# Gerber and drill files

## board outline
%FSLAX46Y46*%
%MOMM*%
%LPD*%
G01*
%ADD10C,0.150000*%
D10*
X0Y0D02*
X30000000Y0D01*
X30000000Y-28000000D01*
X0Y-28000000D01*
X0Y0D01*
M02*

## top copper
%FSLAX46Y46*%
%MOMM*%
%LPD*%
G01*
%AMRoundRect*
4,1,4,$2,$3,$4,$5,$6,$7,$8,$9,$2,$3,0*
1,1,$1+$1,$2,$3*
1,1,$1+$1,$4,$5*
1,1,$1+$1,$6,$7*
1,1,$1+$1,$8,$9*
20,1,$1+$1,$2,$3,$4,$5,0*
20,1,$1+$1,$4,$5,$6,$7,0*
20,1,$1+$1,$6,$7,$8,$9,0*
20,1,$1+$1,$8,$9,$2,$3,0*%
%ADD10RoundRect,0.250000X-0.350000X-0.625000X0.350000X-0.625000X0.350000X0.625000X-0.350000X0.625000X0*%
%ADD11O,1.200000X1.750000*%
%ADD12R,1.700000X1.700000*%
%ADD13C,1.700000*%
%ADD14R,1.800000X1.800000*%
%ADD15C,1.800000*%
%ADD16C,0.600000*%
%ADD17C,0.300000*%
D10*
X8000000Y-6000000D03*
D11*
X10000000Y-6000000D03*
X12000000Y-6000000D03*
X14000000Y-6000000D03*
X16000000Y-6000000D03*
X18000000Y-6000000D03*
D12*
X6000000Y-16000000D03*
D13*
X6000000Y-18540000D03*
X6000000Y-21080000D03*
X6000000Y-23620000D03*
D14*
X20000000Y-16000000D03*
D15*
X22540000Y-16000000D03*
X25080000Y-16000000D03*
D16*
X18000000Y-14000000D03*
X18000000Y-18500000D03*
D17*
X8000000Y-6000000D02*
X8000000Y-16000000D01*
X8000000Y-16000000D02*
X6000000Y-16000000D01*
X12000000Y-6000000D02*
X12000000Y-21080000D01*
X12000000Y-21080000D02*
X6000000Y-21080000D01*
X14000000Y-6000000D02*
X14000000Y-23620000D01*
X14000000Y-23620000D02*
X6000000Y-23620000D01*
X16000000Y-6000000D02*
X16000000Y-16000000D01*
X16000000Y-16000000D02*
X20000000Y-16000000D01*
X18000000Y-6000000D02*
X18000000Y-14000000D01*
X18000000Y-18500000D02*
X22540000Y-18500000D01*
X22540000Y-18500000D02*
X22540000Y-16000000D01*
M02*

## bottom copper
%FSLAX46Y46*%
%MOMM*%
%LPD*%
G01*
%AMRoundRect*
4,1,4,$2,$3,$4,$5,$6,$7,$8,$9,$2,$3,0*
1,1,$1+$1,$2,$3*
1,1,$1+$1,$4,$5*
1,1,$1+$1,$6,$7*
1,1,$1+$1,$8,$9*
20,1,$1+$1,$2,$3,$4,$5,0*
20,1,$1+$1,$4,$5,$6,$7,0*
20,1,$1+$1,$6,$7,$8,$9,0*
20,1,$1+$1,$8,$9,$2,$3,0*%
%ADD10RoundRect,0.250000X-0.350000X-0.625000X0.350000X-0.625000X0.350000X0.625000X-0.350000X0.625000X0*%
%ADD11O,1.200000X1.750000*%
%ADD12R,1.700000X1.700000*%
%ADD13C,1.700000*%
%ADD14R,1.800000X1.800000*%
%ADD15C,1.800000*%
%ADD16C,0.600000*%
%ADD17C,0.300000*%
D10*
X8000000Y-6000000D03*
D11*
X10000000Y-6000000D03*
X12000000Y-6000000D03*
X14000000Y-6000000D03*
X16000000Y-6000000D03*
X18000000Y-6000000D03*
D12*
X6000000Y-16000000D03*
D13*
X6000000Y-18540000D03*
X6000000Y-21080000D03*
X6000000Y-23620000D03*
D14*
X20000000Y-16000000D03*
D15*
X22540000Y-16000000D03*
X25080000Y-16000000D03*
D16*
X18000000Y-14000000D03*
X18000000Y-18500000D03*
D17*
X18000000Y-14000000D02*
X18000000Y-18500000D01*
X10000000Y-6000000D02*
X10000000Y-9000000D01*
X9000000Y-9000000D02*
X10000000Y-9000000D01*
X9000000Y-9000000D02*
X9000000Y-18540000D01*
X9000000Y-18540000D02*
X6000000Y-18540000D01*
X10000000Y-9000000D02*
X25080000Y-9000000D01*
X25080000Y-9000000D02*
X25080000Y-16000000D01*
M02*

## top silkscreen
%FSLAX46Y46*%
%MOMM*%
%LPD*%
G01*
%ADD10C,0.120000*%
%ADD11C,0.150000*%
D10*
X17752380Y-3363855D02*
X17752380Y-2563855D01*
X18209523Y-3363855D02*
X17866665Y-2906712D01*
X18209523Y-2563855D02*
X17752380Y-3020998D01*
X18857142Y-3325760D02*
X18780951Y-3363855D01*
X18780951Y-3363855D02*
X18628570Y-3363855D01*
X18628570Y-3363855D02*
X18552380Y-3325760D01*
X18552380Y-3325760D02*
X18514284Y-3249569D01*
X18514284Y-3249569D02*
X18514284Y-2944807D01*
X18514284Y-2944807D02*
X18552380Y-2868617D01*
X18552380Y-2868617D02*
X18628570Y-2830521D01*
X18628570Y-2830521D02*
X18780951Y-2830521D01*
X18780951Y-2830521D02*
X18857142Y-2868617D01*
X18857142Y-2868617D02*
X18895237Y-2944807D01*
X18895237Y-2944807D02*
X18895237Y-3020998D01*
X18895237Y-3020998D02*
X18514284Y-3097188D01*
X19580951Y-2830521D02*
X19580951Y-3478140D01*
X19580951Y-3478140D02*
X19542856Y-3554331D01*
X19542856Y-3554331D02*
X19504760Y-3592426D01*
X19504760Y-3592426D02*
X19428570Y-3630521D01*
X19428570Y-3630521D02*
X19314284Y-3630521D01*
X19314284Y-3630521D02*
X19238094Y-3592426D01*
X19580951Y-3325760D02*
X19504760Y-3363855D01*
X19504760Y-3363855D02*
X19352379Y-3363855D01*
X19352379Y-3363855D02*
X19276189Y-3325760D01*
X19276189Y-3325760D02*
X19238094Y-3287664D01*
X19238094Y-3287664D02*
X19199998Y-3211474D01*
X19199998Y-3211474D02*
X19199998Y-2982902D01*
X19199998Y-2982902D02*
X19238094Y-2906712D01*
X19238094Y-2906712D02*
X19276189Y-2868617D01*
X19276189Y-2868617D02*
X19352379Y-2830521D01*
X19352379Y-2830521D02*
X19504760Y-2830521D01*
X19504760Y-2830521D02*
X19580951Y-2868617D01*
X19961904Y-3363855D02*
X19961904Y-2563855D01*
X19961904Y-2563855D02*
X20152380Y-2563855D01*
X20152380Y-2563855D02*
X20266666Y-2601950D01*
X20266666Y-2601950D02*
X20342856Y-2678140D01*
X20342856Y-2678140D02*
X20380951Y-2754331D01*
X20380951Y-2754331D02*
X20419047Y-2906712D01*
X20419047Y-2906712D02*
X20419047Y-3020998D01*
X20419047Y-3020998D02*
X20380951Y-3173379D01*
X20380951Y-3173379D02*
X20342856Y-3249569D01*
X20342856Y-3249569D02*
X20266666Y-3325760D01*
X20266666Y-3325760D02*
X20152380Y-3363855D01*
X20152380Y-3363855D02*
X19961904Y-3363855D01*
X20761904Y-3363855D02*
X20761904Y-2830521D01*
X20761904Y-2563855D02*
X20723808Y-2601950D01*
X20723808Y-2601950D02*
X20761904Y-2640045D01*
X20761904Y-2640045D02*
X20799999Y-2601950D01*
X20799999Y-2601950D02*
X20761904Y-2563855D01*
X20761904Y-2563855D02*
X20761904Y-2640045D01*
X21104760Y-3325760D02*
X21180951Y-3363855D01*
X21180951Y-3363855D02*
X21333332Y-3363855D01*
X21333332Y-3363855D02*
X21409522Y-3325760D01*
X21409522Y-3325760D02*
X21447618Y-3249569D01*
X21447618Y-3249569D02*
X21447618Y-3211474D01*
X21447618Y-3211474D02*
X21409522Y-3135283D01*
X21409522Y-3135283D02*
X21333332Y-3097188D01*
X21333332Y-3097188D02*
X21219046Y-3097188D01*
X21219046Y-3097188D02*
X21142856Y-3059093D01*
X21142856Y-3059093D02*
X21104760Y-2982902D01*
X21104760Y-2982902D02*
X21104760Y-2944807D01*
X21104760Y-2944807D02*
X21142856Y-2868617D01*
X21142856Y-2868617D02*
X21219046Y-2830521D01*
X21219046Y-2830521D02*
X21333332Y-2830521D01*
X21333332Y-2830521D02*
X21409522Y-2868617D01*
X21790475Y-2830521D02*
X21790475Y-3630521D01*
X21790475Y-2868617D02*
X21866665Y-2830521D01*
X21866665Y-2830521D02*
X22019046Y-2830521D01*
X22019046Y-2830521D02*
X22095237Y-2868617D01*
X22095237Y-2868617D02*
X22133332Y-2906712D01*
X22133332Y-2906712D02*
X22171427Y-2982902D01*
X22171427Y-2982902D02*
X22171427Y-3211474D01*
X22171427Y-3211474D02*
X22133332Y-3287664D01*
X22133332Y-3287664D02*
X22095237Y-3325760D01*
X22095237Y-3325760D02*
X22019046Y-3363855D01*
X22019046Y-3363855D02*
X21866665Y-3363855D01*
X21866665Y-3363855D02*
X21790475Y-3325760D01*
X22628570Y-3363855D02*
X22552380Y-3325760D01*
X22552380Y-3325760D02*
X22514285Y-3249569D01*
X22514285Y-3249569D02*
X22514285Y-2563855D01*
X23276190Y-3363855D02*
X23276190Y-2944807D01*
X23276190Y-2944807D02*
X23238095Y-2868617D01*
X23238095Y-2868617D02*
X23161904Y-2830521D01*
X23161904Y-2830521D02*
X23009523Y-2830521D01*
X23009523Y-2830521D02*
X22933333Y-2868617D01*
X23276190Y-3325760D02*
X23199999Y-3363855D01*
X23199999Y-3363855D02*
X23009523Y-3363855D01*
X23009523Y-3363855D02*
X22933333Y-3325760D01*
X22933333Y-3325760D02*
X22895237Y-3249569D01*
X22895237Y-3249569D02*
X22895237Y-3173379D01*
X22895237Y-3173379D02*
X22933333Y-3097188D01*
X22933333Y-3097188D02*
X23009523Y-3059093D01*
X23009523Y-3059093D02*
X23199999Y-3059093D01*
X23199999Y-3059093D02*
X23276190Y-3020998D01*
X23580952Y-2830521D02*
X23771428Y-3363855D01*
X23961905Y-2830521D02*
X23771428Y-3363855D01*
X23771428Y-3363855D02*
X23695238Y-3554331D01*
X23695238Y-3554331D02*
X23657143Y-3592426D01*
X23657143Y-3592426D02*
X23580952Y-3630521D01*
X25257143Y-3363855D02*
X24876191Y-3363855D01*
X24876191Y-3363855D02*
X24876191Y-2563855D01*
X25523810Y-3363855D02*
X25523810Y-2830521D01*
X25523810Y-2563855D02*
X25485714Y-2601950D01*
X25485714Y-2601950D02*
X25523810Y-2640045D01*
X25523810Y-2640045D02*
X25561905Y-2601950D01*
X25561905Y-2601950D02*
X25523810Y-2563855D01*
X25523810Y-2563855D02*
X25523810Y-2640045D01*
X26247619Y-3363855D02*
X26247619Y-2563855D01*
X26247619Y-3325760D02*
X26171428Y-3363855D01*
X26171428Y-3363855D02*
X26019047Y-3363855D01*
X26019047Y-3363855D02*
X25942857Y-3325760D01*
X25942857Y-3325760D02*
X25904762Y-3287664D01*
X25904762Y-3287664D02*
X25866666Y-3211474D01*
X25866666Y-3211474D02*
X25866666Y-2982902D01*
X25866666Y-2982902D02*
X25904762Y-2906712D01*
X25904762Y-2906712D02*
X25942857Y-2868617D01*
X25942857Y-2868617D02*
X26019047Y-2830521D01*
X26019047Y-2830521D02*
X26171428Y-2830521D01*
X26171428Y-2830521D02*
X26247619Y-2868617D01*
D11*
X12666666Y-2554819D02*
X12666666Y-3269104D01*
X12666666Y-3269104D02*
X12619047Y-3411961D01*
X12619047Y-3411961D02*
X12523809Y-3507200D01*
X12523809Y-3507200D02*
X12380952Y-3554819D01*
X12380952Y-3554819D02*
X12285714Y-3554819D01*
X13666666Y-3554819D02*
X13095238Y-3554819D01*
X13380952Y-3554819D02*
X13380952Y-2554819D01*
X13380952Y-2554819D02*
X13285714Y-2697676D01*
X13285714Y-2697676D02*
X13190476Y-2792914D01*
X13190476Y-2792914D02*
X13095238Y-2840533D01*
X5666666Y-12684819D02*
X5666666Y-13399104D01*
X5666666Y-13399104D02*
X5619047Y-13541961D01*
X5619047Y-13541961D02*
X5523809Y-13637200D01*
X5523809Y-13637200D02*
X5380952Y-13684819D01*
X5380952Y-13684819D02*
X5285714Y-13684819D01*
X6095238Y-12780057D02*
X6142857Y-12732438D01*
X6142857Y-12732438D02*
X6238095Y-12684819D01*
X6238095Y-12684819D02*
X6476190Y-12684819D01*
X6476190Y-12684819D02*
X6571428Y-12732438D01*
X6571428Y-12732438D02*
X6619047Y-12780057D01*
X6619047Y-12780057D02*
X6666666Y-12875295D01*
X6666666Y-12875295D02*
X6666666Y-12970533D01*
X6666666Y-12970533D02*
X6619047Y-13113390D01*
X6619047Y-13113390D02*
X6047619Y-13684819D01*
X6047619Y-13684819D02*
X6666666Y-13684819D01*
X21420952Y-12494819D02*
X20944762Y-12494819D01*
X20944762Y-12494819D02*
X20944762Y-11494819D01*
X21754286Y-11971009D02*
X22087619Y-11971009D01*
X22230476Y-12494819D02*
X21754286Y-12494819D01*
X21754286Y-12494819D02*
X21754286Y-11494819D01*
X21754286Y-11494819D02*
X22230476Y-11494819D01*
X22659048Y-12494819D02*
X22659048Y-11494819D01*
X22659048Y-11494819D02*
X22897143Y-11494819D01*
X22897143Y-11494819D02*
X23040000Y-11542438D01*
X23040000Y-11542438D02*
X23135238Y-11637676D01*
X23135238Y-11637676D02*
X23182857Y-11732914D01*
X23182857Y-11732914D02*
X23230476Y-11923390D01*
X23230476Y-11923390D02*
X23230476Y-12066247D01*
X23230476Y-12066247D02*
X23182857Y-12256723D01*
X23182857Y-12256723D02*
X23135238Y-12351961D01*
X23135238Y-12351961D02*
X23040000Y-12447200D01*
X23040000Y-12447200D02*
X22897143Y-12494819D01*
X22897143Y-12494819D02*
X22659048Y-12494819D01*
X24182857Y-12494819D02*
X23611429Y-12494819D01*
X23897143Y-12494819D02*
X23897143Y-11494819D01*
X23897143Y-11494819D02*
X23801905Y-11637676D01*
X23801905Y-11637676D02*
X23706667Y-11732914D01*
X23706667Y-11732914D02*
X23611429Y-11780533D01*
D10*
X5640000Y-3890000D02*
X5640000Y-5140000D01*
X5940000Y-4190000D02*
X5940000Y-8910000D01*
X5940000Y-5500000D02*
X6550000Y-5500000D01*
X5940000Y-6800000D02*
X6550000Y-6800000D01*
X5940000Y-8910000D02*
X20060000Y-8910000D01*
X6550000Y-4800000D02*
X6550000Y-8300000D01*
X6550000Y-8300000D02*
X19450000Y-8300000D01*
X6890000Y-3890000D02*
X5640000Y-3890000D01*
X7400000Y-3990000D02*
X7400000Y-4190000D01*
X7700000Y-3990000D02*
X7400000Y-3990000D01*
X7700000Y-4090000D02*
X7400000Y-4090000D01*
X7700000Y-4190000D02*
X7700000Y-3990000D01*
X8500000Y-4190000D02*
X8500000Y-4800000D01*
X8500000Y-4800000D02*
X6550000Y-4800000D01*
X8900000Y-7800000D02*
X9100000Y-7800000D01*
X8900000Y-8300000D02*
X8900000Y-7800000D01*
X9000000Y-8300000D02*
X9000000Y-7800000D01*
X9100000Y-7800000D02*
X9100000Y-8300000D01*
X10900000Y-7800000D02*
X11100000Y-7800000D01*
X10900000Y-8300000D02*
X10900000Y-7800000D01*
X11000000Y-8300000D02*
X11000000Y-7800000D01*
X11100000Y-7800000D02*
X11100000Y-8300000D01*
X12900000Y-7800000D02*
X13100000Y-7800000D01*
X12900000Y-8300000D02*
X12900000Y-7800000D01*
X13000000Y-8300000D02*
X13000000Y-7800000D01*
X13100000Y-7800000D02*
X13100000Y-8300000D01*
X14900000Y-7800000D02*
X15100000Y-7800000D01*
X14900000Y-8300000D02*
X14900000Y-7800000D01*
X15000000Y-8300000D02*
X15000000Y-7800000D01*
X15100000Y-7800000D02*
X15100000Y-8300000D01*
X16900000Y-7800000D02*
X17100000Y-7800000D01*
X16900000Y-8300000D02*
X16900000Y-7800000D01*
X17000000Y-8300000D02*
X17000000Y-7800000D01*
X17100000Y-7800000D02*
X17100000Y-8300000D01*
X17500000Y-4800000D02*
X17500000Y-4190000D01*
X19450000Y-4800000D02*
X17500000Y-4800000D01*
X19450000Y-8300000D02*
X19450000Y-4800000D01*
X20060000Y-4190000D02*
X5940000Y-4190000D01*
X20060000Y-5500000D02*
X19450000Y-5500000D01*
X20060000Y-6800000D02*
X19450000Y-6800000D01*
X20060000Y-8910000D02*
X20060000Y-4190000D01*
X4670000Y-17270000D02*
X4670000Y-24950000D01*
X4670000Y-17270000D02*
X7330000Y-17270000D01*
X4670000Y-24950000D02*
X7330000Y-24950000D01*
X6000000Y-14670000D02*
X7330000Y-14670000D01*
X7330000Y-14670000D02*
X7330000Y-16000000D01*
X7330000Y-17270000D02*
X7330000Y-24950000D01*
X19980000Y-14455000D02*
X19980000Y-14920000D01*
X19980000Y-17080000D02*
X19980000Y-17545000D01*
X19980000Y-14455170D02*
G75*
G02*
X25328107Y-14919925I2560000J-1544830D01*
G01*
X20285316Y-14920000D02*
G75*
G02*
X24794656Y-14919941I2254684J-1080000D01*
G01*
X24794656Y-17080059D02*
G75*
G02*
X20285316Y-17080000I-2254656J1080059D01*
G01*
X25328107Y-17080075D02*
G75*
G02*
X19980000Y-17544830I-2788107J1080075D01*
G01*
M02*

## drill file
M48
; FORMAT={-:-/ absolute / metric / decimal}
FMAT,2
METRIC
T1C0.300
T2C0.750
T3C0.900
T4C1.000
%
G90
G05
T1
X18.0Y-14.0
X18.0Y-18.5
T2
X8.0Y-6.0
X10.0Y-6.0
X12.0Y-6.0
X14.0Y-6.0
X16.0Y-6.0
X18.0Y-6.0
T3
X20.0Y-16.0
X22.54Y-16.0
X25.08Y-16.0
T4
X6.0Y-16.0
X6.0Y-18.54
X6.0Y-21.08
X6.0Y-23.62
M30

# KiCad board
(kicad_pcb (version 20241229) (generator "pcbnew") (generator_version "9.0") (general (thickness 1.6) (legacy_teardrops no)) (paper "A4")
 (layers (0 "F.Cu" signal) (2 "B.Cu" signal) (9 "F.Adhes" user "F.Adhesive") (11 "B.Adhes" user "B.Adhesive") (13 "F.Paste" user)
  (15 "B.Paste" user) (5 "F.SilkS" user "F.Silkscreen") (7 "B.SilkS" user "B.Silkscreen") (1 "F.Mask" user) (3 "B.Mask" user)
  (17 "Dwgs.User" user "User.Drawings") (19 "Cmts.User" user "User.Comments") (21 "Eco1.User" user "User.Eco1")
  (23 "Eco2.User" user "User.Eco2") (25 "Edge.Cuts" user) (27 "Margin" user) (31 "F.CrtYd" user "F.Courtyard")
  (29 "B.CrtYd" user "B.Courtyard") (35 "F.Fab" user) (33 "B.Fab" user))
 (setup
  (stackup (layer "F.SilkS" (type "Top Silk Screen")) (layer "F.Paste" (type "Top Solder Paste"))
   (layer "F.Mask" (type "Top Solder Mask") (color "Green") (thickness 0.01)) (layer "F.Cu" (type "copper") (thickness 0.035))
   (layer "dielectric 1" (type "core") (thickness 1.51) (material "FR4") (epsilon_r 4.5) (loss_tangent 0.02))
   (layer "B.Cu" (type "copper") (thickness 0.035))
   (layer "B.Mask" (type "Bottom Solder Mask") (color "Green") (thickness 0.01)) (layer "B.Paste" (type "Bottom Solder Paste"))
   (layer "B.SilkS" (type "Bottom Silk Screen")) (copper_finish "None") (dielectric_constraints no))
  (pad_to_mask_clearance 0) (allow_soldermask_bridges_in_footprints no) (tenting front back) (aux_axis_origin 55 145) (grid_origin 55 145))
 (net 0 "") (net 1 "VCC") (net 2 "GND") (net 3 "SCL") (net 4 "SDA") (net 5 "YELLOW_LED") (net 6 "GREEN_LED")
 (gr_rect (start 0 0) (end 30 28) (stroke (width 0.15) (type solid)) (fill no) (layer "Edge.Cuts"))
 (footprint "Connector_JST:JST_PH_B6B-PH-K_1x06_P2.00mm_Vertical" (layer "F.Cu") (at 8 6 0) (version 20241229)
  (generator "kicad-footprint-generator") (layer "F.Cu")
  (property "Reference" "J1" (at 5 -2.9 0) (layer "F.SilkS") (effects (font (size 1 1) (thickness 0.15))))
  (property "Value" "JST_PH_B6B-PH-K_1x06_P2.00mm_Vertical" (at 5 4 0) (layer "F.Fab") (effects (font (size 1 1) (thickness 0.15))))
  (fp_line (start -2.36 -2.11) (end -2.36 -0.86) (stroke (width 0.12) (type solid)) (layer "F.SilkS"))
  (fp_line (start -2.06 -1.81) (end -2.06 2.91) (stroke (width 0.12) (type solid)) (layer "F.SilkS"))
  (fp_line (start -2.06 -0.5) (end -1.45 -0.5) (stroke (width 0.12) (type solid)) (layer "F.SilkS"))
  (fp_line (start -2.06 0.8) (end -1.45 0.8) (stroke (width 0.12) (type solid)) (layer "F.SilkS"))
  (fp_line (start -2.06 2.91) (end 12.06 2.91) (stroke (width 0.12) (type solid)) (layer "F.SilkS"))
  (fp_line (start -1.45 -1.2) (end -1.45 2.3) (stroke (width 0.12) (type solid)) (layer "F.SilkS"))
  (fp_line (start -1.45 2.3) (end 11.45 2.3) (stroke (width 0.12) (type solid)) (layer "F.SilkS"))
  (fp_line (start -1.11 -2.11) (end -2.36 -2.11) (stroke (width 0.12) (type solid)) (layer "F.SilkS"))
  (fp_line (start -0.6 -2.01) (end -0.6 -1.81) (stroke (width 0.12) (type solid)) (layer "F.SilkS"))
  (fp_line (start -0.3 -2.01) (end -0.6 -2.01) (stroke (width 0.12) (type solid)) (layer "F.SilkS"))
  (fp_line (start -0.3 -1.91) (end -0.6 -1.91) (stroke (width 0.12) (type solid)) (layer "F.SilkS"))
  (fp_line (start -0.3 -1.81) (end -0.3 -2.01) (stroke (width 0.12) (type solid)) (layer "F.SilkS"))
  (fp_line (start 0.5 -1.81) (end 0.5 -1.2) (stroke (width 0.12) (type solid)) (layer "F.SilkS"))
  (fp_line (start 0.5 -1.2) (end -1.45 -1.2) (stroke (width 0.12) (type solid)) (layer "F.SilkS"))
  (fp_line (start 0.9 1.8) (end 1.1 1.8) (stroke (width 0.12) (type solid)) (layer "F.SilkS"))
  (fp_line (start 0.9 2.3) (end 0.9 1.8) (stroke (width 0.12) (type solid)) (layer "F.SilkS"))
  (fp_line (start 1 2.3) (end 1 1.8) (stroke (width 0.12) (type solid)) (layer "F.SilkS"))
  (fp_line (start 1.1 1.8) (end 1.1 2.3) (stroke (width 0.12) (type solid)) (layer "F.SilkS"))
  (fp_line (start 2.9 1.8) (end 3.1 1.8) (stroke (width 0.12) (type solid)) (layer "F.SilkS"))
  (fp_line (start 2.9 2.3) (end 2.9 1.8) (stroke (width 0.12) (type solid)) (layer "F.SilkS"))
  (fp_line (start 3 2.3) (end 3 1.8) (stroke (width 0.12) (type solid)) (layer "F.SilkS"))
  (fp_line (start 3.1 1.8) (end 3.1 2.3) (stroke (width 0.12) (type solid)) (layer "F.SilkS"))
  (fp_line (start 4.9 1.8) (end 5.1 1.8) (stroke (width 0.12) (type solid)) (layer "F.SilkS"))
  (fp_line (start 4.9 2.3) (end 4.9 1.8) (stroke (width 0.12) (type solid)) (layer "F.SilkS"))
  (fp_line (start 5 2.3) (end 5 1.8) (stroke (width 0.12) (type solid)) (layer "F.SilkS"))
  (fp_line (start 5.1 1.8) (end 5.1 2.3) (stroke (width 0.12) (type solid)) (layer "F.SilkS"))
  (fp_line (start 6.9 1.8) (end 7.1 1.8) (stroke (width 0.12) (type solid)) (layer "F.SilkS"))
  (fp_line (start 6.9 2.3) (end 6.9 1.8) (stroke (width 0.12) (type solid)) (layer "F.SilkS"))
  (fp_line (start 7 2.3) (end 7 1.8) (stroke (width 0.12) (type solid)) (layer "F.SilkS"))
  (fp_line (start 7.1 1.8) (end 7.1 2.3) (stroke (width 0.12) (type solid)) (layer "F.SilkS"))
  (fp_line (start 8.9 1.8) (end 9.1 1.8) (stroke (width 0.12) (type solid)) (layer "F.SilkS"))
  (fp_line (start 8.9 2.3) (end 8.9 1.8) (stroke (width 0.12) (type solid)) (layer "F.SilkS"))
  (fp_line (start 9 2.3) (end 9 1.8) (stroke (width 0.12) (type solid)) (layer "F.SilkS"))
  (fp_line (start 9.1 1.8) (end 9.1 2.3) (stroke (width 0.12) (type solid)) (layer "F.SilkS"))
  (fp_line (start 9.5 -1.2) (end 9.5 -1.81) (stroke (width 0.12) (type solid)) (layer "F.SilkS"))
  (fp_line (start 11.45 -1.2) (end 9.5 -1.2) (stroke (width 0.12) (type solid)) (layer "F.SilkS"))
  (fp_line (start 11.45 2.3) (end 11.45 -1.2) (stroke (width 0.12) (type solid)) (layer "F.SilkS"))
  (fp_line (start 12.06 -1.81) (end -2.06 -1.81) (stroke (width 0.12) (type solid)) (layer "F.SilkS"))
  (fp_line (start 12.06 -0.5) (end 11.45 -0.5) (stroke (width 0.12) (type solid)) (layer "F.SilkS"))
  (fp_line (start 12.06 0.8) (end 11.45 0.8) (stroke (width 0.12) (type solid)) (layer "F.SilkS"))
  (fp_line (start 12.06 2.91) (end 12.06 -1.81) (stroke (width 0.12) (type solid)) (layer "F.SilkS"))
  (pad "1" thru_hole roundrect (at 0 0) (size 1.2 1.75) (drill 0.75) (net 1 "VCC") (layers "*.Cu" "*.Mask") (remove_unused_layers no)
   (roundrect_rratio 0.208333))
  (pad "2" thru_hole oval (at 2 0) (size 1.2 1.75) (drill 0.75) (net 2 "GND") (layers "*.Cu" "*.Mask") (remove_unused_layers no))
  (pad "3" thru_hole oval (at 4 0) (size 1.2 1.75) (drill 0.75) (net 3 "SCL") (layers "*.Cu" "*.Mask") (remove_unused_layers no))
  (pad "4" thru_hole oval (at 6 0) (size 1.2 1.75) (drill 0.75) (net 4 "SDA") (layers "*.Cu" "*.Mask") (remove_unused_layers no))
  (pad "5" thru_hole oval (at 8 0) (size 1.2 1.75) (drill 0.75) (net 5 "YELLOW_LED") (layers "*.Cu" "*.Mask") (remove_unused_layers no))
  (pad "6" thru_hole oval (at 10 0) (size 1.2 1.75) (drill 0.75) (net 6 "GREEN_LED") (layers "*.Cu" "*.Mask") (remove_unused_layers no)))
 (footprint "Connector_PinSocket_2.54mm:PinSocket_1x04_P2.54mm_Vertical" (layer "F.Cu") (at 6 16 0) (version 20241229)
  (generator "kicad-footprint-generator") (layer "F.Cu")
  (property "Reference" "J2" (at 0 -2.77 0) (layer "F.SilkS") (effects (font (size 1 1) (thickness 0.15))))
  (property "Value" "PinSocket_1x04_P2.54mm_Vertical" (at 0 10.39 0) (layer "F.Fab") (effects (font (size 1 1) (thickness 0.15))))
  (fp_line (start -1.33 1.27) (end -1.33 8.95) (stroke (width 0.12) (type solid)) (layer "F.SilkS"))
  (fp_line (start -1.33 1.27) (end 1.33 1.27) (stroke (width 0.12) (type solid)) (layer "F.SilkS"))
  (fp_line (start -1.33 8.95) (end 1.33 8.95) (stroke (width 0.12) (type solid)) (layer "F.SilkS"))
  (fp_line (start 0 -1.33) (end 1.33 -1.33) (stroke (width 0.12) (type solid)) (layer "F.SilkS"))
  (fp_line (start 1.33 -1.33) (end 1.33 0) (stroke (width 0.12) (type solid)) (layer "F.SilkS"))
  (fp_line (start 1.33 1.27) (end 1.33 8.95) (stroke (width 0.12) (type solid)) (layer "F.SilkS"))
  (pad "1" thru_hole rect (at 0 0) (size 1.7 1.7) (drill 1) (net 1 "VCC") (layers "*.Cu" "*.Mask") (remove_unused_layers no))
  (pad "2" thru_hole circle (at 0 2.54) (size 1.7 1.7) (drill 1) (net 2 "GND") (layers "*.Cu" "*.Mask") (remove_unused_layers no))
  (pad "3" thru_hole circle (at 0 5.08) (size 1.7 1.7) (drill 1) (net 3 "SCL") (layers "*.Cu" "*.Mask") (remove_unused_layers no))
  (pad "4" thru_hole circle (at 0 7.62) (size 1.7 1.7) (drill 1) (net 4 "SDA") (layers "*.Cu" "*.Mask") (remove_unused_layers no)))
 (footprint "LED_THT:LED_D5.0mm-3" (layer "F.Cu") (at 20 16 0) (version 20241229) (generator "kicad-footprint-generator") (layer "F.Cu")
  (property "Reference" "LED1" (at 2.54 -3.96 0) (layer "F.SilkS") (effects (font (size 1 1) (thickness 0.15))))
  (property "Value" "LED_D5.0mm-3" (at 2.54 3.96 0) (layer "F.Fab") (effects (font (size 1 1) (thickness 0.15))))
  (fp_line (start -0.02 -1.545) (end -0.02 -1.08) (stroke (width 0.12) (type solid)) (layer "F.SilkS"))
  (fp_line (start -0.02 1.08) (end -0.02 1.545) (stroke (width 0.12) (type solid)) (layer "F.SilkS"))
  (fp_arc (start -0.02 -1.54483) (mid 2.798858 -2.978774) (end 5.328107 -1.080075) (stroke (width 0.12) (type solid)) (layer "F.SilkS"))
  (fp_arc (start 0.285316 -1.08) (mid 2.539967 -2.5) (end 4.794656 -1.080059) (stroke (width 0.12) (type solid)) (layer "F.SilkS"))
  (fp_arc (start 4.794656 1.080059) (mid 2.539967 2.5) (end 0.285316 1.08) (stroke (width 0.12) (type solid)) (layer "F.SilkS"))
  (fp_arc (start 5.328107 1.080075) (mid 2.798858 2.978774) (end -0.02 1.54483) (stroke (width 0.12) (type solid)) (layer "F.SilkS"))
  (pad "1" thru_hole rect (at 0 0) (size 1.8 1.8) (drill 0.9) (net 5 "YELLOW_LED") (layers "*.Cu" "*.Mask") (remove_unused_layers no))
  (pad "2" thru_hole circle (at 2.54 0) (size 1.8 1.8) (drill 0.9) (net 6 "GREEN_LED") (layers "*.Cu" "*.Mask") (remove_unused_layers no))
  (pad "3" thru_hole circle (at 5.08 0) (size 1.8 1.8) (drill 0.9) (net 2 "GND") (layers "*.Cu" "*.Mask") (remove_unused_layers no)))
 (segment (start 8 6) (end 8 16) (width 0.3) (layer "F.Cu") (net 1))
 (segment (start 8 16) (end 6 16) (width 0.3) (layer "F.Cu") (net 1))
 (segment (start 12 6) (end 12 21.08) (width 0.3) (layer "F.Cu") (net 3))
 (segment (start 12 21.08) (end 6 21.08) (width 0.3) (layer "F.Cu") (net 3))
 (segment (start 14 6) (end 14 23.62) (width 0.3) (layer "F.Cu") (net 4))
 (segment (start 14 23.62) (end 6 23.62) (width 0.3) (layer "F.Cu") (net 4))
 (segment (start 16 6) (end 16 16) (width 0.3) (layer "F.Cu") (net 5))
 (segment (start 16 16) (end 20 16) (width 0.3) (layer "F.Cu") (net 5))
 (segment (start 18 6) (end 18 14) (width 0.3) (layer "F.Cu") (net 6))
 (segment (start 18 14) (end 18 18.5) (width 0.3) (layer "B.Cu") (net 6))
 (segment (start 18 18.5) (end 22.54 18.5) (width 0.3) (layer "F.Cu") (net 6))
 (segment (start 22.54 18.5) (end 22.54 16) (width 0.3) (layer "F.Cu") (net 6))
 (segment (start 10 6) (end 10 9) (width 0.3) (layer "B.Cu") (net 2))
 (segment (start 9 9) (end 10 9) (width 0.3) (layer "B.Cu") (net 2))
 (segment (start 9 9) (end 9 18.54) (width 0.3) (layer "B.Cu") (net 2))
 (segment (start 9 18.54) (end 6 18.54) (width 0.3) (layer "B.Cu") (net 2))
 (segment (start 10 9) (end 25.08 9) (width 0.3) (layer "B.Cu") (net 2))
 (segment (start 25.08 9) (end 25.08 16) (width 0.3) (layer "B.Cu") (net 2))
 (via (at 18 14) (size 0.6) (drill 0.3) (layers "F.Cu" "B.Cu") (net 6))
 (via (at 18 18.5) (size 0.6) (drill 0.3) (layers "F.Cu" "B.Cu") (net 6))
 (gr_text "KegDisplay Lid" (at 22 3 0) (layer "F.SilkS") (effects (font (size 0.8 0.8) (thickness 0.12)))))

